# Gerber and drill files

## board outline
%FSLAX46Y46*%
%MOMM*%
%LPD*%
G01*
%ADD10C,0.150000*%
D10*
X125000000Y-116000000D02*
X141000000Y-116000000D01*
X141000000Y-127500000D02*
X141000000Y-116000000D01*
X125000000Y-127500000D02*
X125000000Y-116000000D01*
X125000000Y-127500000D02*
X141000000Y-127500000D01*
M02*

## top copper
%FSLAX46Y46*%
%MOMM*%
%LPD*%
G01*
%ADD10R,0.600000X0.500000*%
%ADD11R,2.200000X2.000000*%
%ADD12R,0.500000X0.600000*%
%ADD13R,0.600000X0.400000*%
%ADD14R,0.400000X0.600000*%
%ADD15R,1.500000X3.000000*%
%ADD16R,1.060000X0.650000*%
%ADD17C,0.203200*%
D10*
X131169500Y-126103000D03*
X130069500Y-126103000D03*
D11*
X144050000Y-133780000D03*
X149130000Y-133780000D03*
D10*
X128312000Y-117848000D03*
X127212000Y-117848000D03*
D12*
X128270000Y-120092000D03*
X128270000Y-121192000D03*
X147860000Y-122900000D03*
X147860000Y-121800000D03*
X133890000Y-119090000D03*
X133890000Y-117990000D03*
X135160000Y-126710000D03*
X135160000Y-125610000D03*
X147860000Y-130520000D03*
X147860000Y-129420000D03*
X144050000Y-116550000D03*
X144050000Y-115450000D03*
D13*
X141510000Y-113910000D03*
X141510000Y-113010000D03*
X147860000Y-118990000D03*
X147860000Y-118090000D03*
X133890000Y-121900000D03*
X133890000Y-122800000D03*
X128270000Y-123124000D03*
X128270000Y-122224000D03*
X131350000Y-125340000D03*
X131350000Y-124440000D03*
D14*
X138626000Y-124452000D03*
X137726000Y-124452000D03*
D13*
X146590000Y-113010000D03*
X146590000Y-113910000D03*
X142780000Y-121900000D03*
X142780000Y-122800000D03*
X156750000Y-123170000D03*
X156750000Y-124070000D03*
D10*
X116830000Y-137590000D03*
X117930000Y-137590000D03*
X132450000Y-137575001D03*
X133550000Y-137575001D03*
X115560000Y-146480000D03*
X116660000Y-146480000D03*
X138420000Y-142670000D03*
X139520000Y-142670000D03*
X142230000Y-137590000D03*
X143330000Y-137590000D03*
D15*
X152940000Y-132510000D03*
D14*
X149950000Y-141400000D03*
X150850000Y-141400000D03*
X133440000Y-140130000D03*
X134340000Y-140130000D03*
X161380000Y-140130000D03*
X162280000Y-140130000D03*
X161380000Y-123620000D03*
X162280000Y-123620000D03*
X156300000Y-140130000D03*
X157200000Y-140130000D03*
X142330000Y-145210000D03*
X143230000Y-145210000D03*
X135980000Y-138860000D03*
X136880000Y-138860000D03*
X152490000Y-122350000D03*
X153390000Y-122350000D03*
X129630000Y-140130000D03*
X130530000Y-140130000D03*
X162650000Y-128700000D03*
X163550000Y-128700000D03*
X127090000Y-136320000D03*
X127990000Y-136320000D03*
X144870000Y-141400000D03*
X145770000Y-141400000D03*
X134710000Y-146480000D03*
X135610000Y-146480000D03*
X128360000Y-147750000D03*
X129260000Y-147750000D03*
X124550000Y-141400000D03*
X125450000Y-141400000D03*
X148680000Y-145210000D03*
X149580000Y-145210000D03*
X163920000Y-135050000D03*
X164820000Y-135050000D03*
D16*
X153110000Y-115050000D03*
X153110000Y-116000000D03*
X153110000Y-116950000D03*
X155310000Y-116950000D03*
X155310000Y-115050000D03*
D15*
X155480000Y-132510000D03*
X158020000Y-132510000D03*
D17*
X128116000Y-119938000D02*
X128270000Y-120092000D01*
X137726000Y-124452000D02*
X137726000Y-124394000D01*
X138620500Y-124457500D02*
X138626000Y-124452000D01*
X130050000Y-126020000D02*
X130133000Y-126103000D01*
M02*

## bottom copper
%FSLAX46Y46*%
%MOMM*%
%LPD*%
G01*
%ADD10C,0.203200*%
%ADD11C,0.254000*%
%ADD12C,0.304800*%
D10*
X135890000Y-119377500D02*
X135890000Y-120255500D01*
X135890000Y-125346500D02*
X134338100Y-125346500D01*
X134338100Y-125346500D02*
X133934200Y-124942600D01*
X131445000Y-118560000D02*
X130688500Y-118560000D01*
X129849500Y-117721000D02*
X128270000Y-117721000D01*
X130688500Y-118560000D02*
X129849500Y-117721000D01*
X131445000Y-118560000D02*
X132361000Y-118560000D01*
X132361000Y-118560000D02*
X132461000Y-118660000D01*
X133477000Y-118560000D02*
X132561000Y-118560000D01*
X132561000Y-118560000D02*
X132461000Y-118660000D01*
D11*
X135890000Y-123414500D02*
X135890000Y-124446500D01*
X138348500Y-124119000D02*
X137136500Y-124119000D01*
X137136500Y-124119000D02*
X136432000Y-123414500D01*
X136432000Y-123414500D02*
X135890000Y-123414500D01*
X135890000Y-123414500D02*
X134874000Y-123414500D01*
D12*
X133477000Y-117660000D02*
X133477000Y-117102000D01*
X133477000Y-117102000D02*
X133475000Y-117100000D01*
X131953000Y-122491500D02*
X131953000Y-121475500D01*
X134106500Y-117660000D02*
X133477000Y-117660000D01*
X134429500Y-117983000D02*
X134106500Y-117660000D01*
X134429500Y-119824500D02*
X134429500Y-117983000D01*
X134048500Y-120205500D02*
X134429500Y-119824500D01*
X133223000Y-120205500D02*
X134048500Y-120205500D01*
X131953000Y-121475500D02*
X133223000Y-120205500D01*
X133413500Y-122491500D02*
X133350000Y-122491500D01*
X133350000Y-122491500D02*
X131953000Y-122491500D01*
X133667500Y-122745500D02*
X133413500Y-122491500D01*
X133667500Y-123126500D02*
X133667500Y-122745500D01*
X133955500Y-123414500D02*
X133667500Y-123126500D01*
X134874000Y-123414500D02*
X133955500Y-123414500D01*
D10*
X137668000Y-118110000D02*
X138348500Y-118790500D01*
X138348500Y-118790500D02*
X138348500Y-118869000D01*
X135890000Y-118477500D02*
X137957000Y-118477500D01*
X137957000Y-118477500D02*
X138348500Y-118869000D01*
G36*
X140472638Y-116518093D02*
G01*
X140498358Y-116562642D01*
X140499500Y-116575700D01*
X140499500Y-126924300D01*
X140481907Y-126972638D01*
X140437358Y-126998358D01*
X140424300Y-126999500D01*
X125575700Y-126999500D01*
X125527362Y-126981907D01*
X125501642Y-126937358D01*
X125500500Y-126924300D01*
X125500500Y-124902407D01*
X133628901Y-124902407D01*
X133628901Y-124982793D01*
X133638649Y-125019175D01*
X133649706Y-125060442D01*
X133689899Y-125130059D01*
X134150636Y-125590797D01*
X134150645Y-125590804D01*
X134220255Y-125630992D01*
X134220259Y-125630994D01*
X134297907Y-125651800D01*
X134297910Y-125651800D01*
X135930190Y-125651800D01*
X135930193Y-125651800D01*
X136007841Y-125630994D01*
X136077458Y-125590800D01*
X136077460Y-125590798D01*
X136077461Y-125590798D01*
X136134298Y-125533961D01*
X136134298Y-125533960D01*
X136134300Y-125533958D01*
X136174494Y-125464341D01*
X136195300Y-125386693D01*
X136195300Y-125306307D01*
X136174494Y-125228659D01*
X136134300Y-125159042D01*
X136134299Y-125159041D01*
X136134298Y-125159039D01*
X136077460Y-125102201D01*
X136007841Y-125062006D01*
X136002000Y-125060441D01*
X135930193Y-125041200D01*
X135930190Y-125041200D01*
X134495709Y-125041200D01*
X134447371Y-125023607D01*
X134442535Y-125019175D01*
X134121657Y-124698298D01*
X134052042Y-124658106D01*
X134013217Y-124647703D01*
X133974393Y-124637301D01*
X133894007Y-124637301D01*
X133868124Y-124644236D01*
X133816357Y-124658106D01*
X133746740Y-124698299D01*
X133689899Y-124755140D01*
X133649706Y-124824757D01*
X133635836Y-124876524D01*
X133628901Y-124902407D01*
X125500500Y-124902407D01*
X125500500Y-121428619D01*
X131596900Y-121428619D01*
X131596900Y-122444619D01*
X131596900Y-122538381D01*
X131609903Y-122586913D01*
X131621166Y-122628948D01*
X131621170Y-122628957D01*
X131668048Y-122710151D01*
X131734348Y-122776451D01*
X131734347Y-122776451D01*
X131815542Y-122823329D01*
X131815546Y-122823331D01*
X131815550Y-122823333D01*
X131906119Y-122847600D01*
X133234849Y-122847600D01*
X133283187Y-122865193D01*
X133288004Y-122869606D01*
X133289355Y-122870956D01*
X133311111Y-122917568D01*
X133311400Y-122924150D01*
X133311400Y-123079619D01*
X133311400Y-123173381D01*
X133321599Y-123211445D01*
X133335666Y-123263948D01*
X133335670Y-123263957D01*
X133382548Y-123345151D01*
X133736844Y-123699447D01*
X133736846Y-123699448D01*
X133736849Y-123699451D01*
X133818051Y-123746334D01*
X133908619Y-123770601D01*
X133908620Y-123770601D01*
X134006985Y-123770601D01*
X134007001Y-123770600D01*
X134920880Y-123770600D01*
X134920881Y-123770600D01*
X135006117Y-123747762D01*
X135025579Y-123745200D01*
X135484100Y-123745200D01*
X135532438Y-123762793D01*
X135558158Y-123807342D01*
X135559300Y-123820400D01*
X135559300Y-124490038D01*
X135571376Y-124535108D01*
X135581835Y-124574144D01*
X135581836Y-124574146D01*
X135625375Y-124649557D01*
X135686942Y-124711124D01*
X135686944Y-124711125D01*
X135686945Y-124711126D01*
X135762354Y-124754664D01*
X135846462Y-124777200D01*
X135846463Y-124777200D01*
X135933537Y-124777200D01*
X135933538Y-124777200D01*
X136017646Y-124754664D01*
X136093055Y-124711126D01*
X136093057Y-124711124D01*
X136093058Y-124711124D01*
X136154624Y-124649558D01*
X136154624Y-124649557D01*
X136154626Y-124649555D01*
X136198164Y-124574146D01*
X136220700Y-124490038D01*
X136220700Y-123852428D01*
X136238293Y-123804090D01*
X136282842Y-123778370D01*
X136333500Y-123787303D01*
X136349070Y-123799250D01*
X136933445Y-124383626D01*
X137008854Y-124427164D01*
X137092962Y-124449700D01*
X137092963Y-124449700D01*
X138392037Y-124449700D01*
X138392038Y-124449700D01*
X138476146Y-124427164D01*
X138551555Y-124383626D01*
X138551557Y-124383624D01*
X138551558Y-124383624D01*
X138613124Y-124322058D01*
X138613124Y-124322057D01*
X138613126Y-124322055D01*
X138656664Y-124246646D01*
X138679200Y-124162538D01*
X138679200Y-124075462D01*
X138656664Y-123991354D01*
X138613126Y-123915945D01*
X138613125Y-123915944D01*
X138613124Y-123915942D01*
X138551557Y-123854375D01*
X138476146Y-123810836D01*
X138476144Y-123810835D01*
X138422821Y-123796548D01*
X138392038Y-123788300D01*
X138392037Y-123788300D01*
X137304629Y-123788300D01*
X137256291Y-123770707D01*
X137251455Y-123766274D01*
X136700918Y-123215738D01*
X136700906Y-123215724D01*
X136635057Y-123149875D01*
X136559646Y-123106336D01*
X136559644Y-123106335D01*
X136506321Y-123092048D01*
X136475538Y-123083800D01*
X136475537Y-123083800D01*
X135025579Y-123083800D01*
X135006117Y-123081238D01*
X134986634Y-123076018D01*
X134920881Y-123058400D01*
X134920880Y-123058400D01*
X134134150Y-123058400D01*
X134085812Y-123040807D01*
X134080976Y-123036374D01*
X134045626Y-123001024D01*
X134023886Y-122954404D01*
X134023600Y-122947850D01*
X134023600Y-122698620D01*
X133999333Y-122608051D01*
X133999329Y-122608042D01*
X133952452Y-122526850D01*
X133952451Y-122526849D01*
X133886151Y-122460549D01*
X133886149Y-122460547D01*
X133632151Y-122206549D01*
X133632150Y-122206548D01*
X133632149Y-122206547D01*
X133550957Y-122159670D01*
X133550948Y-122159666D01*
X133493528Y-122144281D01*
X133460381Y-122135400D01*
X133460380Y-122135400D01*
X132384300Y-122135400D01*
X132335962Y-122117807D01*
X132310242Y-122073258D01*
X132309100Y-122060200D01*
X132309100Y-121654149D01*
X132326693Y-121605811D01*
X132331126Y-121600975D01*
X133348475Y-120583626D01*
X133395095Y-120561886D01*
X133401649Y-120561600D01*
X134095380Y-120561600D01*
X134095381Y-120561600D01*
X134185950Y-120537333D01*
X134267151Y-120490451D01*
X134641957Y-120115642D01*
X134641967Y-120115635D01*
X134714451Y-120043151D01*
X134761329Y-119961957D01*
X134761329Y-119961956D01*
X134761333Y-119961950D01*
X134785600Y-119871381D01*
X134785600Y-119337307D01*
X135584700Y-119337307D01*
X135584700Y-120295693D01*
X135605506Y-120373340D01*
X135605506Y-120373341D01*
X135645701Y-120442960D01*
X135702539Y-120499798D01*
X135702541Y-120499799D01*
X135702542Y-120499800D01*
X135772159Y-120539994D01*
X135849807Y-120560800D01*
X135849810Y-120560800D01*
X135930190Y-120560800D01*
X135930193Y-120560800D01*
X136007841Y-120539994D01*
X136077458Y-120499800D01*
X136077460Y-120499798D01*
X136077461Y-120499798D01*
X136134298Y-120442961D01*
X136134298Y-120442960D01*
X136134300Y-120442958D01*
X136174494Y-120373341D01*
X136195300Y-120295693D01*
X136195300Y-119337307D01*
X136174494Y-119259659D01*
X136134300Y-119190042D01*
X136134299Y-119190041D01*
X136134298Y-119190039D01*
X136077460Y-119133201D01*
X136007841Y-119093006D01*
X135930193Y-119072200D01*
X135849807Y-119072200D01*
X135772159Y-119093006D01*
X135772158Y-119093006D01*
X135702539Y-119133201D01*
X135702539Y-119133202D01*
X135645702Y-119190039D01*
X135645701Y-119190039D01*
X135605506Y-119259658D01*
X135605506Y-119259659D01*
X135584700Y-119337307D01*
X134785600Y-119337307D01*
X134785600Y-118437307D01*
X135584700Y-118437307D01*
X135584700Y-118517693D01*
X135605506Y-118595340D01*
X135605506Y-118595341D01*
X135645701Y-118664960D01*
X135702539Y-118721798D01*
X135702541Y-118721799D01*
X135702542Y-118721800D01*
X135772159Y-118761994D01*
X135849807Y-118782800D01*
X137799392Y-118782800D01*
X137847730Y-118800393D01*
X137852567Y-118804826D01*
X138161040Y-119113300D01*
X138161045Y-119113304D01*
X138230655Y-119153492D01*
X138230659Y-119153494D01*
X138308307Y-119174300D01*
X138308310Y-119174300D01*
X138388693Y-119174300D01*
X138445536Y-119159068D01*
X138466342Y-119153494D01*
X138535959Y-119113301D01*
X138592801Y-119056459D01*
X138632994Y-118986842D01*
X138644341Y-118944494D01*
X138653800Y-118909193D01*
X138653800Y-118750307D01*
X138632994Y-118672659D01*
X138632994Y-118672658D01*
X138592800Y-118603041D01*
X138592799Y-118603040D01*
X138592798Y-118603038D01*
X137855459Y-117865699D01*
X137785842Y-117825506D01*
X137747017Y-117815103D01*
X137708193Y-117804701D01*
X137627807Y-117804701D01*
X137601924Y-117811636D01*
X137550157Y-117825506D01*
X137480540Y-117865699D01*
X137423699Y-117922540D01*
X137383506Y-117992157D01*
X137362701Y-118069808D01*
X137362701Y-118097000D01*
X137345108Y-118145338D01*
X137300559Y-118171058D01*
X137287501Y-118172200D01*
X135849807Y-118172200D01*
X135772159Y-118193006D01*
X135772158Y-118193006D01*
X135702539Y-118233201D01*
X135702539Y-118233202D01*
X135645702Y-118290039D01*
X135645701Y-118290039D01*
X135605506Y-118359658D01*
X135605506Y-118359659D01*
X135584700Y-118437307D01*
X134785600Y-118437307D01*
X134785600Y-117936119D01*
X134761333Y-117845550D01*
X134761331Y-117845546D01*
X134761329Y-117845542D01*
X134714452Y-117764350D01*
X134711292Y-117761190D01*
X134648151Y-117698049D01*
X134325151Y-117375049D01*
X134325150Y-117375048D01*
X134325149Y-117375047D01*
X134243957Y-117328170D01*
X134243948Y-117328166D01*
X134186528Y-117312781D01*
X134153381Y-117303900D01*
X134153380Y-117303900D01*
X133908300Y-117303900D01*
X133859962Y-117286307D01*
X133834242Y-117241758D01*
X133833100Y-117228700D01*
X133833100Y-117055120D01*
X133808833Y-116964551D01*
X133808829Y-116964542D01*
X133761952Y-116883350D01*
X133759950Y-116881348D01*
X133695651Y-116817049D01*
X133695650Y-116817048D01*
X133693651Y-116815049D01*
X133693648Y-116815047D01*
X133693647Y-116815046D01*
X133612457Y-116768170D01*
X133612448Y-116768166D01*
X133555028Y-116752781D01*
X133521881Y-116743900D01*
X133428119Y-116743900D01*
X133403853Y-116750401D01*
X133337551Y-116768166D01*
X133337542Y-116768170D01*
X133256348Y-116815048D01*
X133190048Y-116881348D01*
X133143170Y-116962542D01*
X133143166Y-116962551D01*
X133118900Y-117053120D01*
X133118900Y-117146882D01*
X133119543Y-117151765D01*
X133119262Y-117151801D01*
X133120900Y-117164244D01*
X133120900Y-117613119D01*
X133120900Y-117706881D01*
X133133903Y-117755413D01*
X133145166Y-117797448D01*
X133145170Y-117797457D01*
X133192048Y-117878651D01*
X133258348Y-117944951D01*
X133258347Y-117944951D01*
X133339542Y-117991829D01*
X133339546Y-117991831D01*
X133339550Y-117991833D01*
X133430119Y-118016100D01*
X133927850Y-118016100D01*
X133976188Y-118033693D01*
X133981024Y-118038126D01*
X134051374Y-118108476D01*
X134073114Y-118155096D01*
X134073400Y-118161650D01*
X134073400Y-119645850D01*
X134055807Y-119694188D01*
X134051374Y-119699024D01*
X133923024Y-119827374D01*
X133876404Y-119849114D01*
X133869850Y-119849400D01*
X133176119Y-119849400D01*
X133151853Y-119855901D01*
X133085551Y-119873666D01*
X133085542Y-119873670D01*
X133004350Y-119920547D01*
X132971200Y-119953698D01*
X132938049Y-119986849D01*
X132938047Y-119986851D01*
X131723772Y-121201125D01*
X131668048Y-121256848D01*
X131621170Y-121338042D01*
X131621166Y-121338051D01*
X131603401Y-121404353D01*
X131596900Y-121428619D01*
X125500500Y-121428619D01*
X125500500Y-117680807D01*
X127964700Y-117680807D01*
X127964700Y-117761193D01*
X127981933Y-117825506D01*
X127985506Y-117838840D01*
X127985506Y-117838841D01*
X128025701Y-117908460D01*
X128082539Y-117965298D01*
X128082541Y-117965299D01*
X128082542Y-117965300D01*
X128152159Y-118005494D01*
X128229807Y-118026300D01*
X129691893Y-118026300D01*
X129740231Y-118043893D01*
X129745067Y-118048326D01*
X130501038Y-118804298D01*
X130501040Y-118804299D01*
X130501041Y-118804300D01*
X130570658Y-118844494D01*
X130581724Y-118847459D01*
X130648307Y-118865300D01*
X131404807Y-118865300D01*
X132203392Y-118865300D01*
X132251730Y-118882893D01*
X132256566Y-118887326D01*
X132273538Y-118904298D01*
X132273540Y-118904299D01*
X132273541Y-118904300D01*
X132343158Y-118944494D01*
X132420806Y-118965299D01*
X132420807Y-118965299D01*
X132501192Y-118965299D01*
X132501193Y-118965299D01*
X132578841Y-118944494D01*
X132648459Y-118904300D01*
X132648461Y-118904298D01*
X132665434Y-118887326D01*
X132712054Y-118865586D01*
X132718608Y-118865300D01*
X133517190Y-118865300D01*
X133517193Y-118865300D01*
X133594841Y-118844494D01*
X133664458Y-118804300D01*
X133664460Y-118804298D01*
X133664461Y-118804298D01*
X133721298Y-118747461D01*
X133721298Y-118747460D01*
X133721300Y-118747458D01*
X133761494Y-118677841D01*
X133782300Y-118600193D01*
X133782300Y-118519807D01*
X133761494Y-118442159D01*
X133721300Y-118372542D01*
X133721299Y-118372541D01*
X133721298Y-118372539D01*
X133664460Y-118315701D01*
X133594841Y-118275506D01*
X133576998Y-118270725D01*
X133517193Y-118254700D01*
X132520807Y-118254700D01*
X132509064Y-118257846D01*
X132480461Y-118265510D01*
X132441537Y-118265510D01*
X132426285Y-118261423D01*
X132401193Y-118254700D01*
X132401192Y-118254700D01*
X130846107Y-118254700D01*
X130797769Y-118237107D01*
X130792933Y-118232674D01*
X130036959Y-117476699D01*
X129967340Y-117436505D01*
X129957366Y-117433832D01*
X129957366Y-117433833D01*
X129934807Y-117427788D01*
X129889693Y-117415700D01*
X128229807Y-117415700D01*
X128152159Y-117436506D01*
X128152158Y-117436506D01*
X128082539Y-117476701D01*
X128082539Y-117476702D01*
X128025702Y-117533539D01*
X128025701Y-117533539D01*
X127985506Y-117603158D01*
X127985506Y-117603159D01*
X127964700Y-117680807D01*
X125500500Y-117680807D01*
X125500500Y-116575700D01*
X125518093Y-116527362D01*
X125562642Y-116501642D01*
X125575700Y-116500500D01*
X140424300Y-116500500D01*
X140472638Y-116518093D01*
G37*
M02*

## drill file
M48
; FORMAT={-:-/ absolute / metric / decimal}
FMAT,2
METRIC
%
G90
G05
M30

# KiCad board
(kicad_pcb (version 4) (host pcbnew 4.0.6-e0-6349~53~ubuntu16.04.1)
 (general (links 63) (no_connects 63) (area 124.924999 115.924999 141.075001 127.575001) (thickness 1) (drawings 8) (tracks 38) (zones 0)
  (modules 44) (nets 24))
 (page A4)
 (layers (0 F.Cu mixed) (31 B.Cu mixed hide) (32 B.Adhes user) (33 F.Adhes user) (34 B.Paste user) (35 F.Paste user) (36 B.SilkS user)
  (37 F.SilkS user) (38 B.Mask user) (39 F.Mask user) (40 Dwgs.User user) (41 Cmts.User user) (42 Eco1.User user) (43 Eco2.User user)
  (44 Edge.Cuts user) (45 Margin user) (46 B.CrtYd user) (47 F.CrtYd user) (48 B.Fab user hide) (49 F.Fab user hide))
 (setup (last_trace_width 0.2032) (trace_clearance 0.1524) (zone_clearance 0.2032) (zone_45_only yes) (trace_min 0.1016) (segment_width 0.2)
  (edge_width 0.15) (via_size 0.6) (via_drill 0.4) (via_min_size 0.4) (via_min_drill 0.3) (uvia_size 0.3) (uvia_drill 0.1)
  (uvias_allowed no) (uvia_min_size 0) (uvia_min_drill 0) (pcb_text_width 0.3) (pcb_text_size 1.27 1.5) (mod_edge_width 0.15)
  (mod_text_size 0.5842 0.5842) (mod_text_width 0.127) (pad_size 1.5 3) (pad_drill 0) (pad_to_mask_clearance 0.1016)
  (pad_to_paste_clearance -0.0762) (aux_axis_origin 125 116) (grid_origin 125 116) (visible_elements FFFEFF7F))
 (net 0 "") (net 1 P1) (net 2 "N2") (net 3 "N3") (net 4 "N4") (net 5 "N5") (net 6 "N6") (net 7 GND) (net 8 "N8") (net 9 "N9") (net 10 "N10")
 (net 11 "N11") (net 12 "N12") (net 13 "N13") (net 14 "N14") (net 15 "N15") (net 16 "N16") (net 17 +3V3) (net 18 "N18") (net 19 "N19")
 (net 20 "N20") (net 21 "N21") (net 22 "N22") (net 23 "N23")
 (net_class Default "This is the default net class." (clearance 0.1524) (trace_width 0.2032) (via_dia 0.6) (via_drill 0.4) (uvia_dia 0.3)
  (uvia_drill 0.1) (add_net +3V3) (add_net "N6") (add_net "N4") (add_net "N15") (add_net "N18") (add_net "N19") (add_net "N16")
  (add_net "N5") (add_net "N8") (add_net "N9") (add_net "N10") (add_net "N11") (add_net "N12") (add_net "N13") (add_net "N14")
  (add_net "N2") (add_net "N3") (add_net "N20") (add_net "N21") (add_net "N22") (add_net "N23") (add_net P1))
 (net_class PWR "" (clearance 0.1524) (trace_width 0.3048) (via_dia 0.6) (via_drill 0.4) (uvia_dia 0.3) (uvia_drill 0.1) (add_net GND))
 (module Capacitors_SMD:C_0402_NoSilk (layer F.Cu) (at 130.6195 126.103 180)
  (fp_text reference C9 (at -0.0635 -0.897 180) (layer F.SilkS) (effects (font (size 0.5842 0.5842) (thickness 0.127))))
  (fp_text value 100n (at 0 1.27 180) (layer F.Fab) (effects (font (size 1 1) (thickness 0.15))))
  (pad 1 smd rect (at -0.55 0 180) (size 0.6 0.5) (layers F.Cu F.Paste F.Mask) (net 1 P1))
  (pad 2 smd rect (at 0.55 0 180) (size 0.6 0.5) (layers F.Cu F.Paste F.Mask) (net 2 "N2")))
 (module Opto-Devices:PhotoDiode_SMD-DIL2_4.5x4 (layer F.Cu) (at 146.59 133.78 180)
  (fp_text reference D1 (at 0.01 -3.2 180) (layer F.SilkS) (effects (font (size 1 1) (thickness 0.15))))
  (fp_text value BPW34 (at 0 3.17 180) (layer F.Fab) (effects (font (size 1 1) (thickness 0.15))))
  (pad 2 smd rect (at 2.54 0) (size 2.2 2) (layers F.Cu F.Paste F.Mask) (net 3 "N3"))
  (pad 1 smd rect (at -2.54 0) (size 2.2 2) (layers F.Cu F.Paste F.Mask) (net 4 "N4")))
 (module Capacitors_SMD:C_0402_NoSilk (layer F.Cu) (at 127.762 117.848 180)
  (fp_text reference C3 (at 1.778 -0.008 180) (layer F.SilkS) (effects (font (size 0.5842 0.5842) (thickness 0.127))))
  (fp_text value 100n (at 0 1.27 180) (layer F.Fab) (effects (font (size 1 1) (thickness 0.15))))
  (pad 1 smd rect (at -0.55 0 180) (size 0.6 0.5) (layers F.Cu F.Paste F.Mask) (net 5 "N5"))
  (pad 2 smd rect (at 0.55 0 180) (size 0.6 0.5) (layers F.Cu F.Paste F.Mask) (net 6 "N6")))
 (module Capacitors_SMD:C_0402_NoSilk (layer F.Cu) (at 128.27 120.642 270)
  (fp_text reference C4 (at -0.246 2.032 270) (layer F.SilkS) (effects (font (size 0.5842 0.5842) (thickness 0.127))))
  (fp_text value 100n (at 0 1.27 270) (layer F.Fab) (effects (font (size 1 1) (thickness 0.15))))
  (pad 1 smd rect (at -0.55 0 270) (size 0.6 0.5) (layers F.Cu F.Paste F.Mask) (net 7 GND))
  (pad 2 smd rect (at 0.55 0 270) (size 0.6 0.5) (layers F.Cu F.Paste F.Mask) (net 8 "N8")))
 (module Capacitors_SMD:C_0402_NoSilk (layer F.Cu) (at 147.86 122.35 90)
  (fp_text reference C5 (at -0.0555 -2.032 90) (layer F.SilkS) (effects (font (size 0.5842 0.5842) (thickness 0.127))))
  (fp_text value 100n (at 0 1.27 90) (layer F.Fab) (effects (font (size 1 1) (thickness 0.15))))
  (pad 1 smd rect (at -0.55 0 90) (size 0.6 0.5) (layers F.Cu F.Paste F.Mask) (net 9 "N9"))
  (pad 2 smd rect (at 0.55 0 90) (size 0.6 0.5) (layers F.Cu F.Paste F.Mask) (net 7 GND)))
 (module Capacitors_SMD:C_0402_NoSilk (layer F.Cu) (at 133.89 118.54 90)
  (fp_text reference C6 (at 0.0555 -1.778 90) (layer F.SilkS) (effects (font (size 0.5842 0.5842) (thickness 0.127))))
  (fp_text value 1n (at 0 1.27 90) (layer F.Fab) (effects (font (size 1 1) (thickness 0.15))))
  (pad 1 smd rect (at -0.55 0 90) (size 0.6 0.5) (layers F.Cu F.Paste F.Mask) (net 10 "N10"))
  (pad 2 smd rect (at 0.55 0 90) (size 0.6 0.5) (layers F.Cu F.Paste F.Mask) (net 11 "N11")))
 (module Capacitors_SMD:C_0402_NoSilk (layer F.Cu) (at 135.16 126.16 90)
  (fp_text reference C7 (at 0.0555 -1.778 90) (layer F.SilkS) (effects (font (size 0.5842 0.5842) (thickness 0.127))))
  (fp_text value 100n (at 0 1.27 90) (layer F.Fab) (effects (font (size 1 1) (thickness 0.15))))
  (pad 1 smd rect (at -0.55 0 90) (size 0.6 0.5) (layers F.Cu F.Paste F.Mask) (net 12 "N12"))
  (pad 2 smd rect (at 0.55 0 90) (size 0.6 0.5) (layers F.Cu F.Paste F.Mask) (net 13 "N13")))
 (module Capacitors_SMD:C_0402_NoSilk (layer F.Cu) (at 147.86 129.97 90)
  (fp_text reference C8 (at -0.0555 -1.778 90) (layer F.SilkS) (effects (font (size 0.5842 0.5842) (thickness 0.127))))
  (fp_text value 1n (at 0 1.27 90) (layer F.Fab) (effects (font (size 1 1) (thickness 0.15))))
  (pad 1 smd rect (at -0.55 0 90) (size 0.6 0.5) (layers F.Cu F.Paste F.Mask) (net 7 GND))
  (pad 2 smd rect (at 0.55 0 90) (size 0.6 0.5) (layers F.Cu F.Paste F.Mask) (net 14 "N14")))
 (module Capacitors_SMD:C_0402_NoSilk (layer F.Cu) (at 144.05 116 90)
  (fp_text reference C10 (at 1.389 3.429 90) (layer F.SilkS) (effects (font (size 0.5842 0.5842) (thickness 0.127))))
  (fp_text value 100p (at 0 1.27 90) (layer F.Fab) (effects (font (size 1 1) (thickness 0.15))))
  (pad 1 smd rect (at -0.55 0 90) (size 0.6 0.5) (layers F.Cu F.Paste F.Mask) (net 7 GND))
  (pad 2 smd rect (at 0.55 0 90) (size 0.6 0.5) (layers F.Cu F.Paste F.Mask) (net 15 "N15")))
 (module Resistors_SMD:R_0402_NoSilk (layer F.Cu) (at 141.51 113.46 90)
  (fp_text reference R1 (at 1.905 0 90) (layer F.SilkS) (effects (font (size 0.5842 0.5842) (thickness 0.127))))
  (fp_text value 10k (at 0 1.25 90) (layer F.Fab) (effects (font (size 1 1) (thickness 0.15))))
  (pad 1 smd rect (at -0.45 0 90) (size 0.4 0.6) (layers F.Cu F.Paste F.Mask) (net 8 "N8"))
  (pad 2 smd rect (at 0.45 0 90) (size 0.4 0.6) (layers F.Cu F.Paste F.Mask) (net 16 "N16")))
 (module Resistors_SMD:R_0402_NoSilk (layer F.Cu) (at 147.86 118.54 90)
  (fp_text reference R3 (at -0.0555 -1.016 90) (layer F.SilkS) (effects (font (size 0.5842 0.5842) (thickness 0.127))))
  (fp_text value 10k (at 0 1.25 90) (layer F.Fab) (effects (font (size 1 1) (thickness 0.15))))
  (pad 1 smd rect (at -0.45 0 90) (size 0.4 0.6) (layers F.Cu F.Paste F.Mask) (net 16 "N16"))
  (pad 2 smd rect (at 0.45 0 90) (size 0.4 0.6) (layers F.Cu F.Paste F.Mask) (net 4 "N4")))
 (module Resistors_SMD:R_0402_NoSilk (layer F.Cu) (at 133.89 122.35 270)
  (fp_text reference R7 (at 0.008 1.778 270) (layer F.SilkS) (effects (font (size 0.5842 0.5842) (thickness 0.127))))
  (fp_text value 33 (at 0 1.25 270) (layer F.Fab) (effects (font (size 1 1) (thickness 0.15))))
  (pad 1 smd rect (at -0.45 0 270) (size 0.4 0.6) (layers F.Cu F.Paste F.Mask) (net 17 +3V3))
  (pad 2 smd rect (at 0.45 0 270) (size 0.4 0.6) (layers F.Cu F.Paste F.Mask) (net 8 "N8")))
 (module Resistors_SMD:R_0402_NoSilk (layer F.Cu) (at 128.27 122.674 90)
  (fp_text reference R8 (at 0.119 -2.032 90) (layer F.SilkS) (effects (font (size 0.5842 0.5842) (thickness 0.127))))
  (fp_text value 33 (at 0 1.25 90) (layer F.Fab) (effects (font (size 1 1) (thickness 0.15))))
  (pad 1 smd rect (at -0.45 0 90) (size 0.4 0.6) (layers F.Cu F.Paste F.Mask) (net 17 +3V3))
  (pad 2 smd rect (at 0.45 0 90) (size 0.4 0.6) (layers F.Cu F.Paste F.Mask) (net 9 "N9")))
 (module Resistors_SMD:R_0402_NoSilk (layer F.Cu) (at 131.35 124.89 90)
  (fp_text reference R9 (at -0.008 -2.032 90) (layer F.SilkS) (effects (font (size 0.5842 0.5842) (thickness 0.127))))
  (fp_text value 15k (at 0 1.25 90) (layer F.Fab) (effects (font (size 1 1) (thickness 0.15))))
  (pad 1 smd rect (at -0.45 0 90) (size 0.4 0.6) (layers F.Cu F.Paste F.Mask) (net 9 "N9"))
  (pad 2 smd rect (at 0.45 0 90) (size 0.4 0.6) (layers F.Cu F.Paste F.Mask) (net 5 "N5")))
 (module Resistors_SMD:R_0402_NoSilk (layer F.Cu) (at 138.176 124.452 180)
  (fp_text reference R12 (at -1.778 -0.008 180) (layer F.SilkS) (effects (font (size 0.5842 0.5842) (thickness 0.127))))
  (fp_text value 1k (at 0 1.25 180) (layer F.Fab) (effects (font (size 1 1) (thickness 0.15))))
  (pad 1 smd rect (at -0.45 0 180) (size 0.4 0.6) (layers F.Cu F.Paste F.Mask) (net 11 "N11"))
  (pad 2 smd rect (at 0.45 0 180) (size 0.4 0.6) (layers F.Cu F.Paste F.Mask) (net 10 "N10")))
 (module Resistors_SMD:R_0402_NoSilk (layer F.Cu) (at 146.59 113.46 270)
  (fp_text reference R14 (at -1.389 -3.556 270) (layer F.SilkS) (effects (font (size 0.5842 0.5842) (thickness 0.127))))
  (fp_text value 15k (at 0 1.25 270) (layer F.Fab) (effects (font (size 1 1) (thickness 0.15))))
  (pad 1 smd rect (at -0.45 0 270) (size 0.4 0.6) (layers F.Cu F.Paste F.Mask) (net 12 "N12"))
  (pad 2 smd rect (at 0.45 0 270) (size 0.4 0.6) (layers F.Cu F.Paste F.Mask) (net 10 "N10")))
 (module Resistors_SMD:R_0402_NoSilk (layer F.Cu) (at 142.78 122.35 270)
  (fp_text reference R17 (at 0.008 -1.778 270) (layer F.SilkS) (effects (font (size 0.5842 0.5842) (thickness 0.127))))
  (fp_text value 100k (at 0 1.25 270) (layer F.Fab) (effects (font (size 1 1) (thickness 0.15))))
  (pad 1 smd rect (at -0.45 0 270) (size 0.4 0.6) (layers F.Cu F.Paste F.Mask) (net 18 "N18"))
  (pad 2 smd rect (at 0.45 0 270) (size 0.4 0.6) (layers F.Cu F.Paste F.Mask) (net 1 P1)))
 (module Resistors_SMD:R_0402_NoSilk (layer F.Cu) (at 156.75 123.62 270)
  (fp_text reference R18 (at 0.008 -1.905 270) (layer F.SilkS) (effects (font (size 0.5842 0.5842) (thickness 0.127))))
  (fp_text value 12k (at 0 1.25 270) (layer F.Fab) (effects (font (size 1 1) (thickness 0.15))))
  (pad 1 smd rect (at -0.45 0 270) (size 0.4 0.6) (layers F.Cu F.Paste F.Mask) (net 1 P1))
  (pad 2 smd rect (at 0.45 0 270) (size 0.4 0.6) (layers F.Cu F.Paste F.Mask) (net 7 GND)))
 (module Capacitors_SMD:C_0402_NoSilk (layer F.Cu) (at 117.38 137.59)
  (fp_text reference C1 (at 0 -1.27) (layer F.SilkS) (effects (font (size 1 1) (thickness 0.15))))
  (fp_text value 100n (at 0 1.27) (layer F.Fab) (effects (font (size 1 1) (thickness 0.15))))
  (pad 1 smd rect (at -0.55 0) (size 0.6 0.5) (layers F.Cu F.Paste F.Mask) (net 6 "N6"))
  (pad 2 smd rect (at 0.55 0) (size 0.6 0.5) (layers F.Cu F.Paste F.Mask) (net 4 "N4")))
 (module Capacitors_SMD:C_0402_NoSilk (layer F.Cu) (at 133 137.575001)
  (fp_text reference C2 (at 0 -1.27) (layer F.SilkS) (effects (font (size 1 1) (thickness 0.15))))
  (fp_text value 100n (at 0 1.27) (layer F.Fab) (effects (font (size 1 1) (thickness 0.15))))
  (pad 1 smd rect (at -0.55 0) (size 0.6 0.5) (layers F.Cu F.Paste F.Mask) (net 16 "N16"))
  (pad 2 smd rect (at 0.55 0) (size 0.6 0.5) (layers F.Cu F.Paste F.Mask) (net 7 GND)))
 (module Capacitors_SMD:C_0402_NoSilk (layer F.Cu) (at 116.11 146.48)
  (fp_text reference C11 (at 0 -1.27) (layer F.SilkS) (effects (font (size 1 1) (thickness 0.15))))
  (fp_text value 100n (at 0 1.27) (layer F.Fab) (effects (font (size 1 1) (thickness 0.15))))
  (pad 1 smd rect (at -0.55 0) (size 0.6 0.5) (layers F.Cu F.Paste F.Mask) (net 7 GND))
  (pad 2 smd rect (at 0.55 0) (size 0.6 0.5) (layers F.Cu F.Paste F.Mask) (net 18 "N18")))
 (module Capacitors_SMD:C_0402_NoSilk (layer F.Cu) (at 138.97 142.67)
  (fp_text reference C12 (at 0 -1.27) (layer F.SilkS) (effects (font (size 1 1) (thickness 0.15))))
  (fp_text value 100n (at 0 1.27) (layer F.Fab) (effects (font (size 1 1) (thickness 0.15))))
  (pad 1 smd rect (at -0.55 0) (size 0.6 0.5) (layers F.Cu F.Paste F.Mask) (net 7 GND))
  (pad 2 smd rect (at 0.55 0) (size 0.6 0.5) (layers F.Cu F.Paste F.Mask) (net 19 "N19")))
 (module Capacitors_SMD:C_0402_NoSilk (layer F.Cu) (at 142.78 137.59)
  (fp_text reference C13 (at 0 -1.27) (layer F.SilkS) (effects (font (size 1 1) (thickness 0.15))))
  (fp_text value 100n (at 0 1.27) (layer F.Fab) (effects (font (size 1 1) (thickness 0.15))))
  (pad 1 smd rect (at -0.55 0) (size 0.6 0.5) (layers F.Cu F.Paste F.Mask) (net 7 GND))
  (pad 2 smd rect (at 0.55 0) (size 0.6 0.5) (layers F.Cu F.Paste F.Mask) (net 17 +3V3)))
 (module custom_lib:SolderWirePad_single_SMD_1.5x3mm (layer F.Cu) (at 152.94 132.51)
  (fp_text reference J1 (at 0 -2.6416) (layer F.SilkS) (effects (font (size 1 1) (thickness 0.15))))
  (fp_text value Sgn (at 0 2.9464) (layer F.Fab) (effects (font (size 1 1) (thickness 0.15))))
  (pad 1 smd rect (at 0 0) (size 1.5 3) (layers F.Cu F.Paste F.Mask) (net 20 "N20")))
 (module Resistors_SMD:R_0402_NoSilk (layer F.Cu) (at 150.4 141.4)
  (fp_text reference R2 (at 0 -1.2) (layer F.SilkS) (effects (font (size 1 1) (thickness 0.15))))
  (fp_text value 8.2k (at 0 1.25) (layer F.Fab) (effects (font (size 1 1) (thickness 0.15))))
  (pad 1 smd rect (at -0.45 0) (size 0.4 0.6) (layers F.Cu F.Paste F.Mask) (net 8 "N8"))
  (pad 2 smd rect (at 0.45 0) (size 0.4 0.6) (layers F.Cu F.Paste F.Mask) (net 3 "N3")))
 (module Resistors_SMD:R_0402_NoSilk (layer F.Cu) (at 133.89 140.13)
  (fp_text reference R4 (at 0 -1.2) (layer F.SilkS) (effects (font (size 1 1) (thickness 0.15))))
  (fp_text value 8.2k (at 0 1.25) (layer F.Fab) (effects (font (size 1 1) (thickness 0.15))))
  (pad 1 smd rect (at -0.45 0) (size 0.4 0.6) (layers F.Cu F.Paste F.Mask) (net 3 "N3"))
  (pad 2 smd rect (at 0.45 0) (size 0.4 0.6) (layers F.Cu F.Paste F.Mask) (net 7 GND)))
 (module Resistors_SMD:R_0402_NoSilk (layer F.Cu) (at 161.83 140.13)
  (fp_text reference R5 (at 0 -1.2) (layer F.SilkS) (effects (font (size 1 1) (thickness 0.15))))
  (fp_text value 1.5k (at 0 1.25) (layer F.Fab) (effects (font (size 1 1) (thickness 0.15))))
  (pad 1 smd rect (at -0.45 0) (size 0.4 0.6) (layers F.Cu F.Paste F.Mask) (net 8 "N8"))
  (pad 2 smd rect (at 0.45 0) (size 0.4 0.6) (layers F.Cu F.Paste F.Mask)))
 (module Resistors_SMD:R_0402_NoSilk (layer F.Cu) (at 161.83 123.62)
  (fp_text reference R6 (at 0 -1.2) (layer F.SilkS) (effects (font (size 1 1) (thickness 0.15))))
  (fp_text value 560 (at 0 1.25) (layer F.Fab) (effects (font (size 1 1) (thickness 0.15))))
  (pad 1 smd rect (at -0.45 0) (size 0.4 0.6) (layers F.Cu F.Paste F.Mask) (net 6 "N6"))
  (pad 2 smd rect (at 0.45 0) (size 0.4 0.6) (layers F.Cu F.Paste F.Mask) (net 7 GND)))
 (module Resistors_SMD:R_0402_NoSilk (layer F.Cu) (at 156.75 140.13)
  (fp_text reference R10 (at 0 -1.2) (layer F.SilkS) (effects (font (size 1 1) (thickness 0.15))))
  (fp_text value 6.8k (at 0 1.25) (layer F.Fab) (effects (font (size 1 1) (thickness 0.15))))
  (pad 1 smd rect (at -0.45 0) (size 0.4 0.6) (layers F.Cu F.Paste F.Mask) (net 5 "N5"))
  (pad 2 smd rect (at 0.45 0) (size 0.4 0.6) (layers F.Cu F.Paste F.Mask) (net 10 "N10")))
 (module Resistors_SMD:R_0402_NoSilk (layer F.Cu) (at 142.78 145.21)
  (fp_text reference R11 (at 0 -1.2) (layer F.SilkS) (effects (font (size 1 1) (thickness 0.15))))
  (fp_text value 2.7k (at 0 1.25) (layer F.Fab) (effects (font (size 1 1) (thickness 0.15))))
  (pad 1 smd rect (at -0.45 0) (size 0.4 0.6) (layers F.Cu F.Paste F.Mask) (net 9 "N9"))
  (pad 2 smd rect (at 0.45 0) (size 0.4 0.6) (layers F.Cu F.Paste F.Mask) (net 13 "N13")))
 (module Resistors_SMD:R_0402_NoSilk (layer F.Cu) (at 136.43 138.86)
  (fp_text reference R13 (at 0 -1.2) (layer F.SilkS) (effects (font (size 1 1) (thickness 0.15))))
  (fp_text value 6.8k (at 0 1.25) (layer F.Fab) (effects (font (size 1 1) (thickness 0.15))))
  (pad 1 smd rect (at -0.45 0) (size 0.4 0.6) (layers F.Cu F.Paste F.Mask) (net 9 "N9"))
  (pad 2 smd rect (at 0.45 0) (size 0.4 0.6) (layers F.Cu F.Paste F.Mask) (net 12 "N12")))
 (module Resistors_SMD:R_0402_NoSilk (layer F.Cu) (at 152.94 122.35)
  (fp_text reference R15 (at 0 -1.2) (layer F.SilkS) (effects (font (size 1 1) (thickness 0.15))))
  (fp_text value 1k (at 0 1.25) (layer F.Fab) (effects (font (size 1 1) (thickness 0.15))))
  (pad 1 smd rect (at -0.45 0) (size 0.4 0.6) (layers F.Cu F.Paste F.Mask) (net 9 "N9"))
  (pad 2 smd rect (at 0.45 0) (size 0.4 0.6) (layers F.Cu F.Paste F.Mask) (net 14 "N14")))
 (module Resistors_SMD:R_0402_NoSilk (layer F.Cu) (at 130.08 140.13)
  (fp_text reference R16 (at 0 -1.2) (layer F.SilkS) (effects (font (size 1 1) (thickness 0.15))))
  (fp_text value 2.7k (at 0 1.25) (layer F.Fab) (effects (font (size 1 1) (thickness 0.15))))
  (pad 1 smd rect (at -0.45 0) (size 0.4 0.6) (layers F.Cu F.Paste F.Mask) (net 2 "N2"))
  (pad 2 smd rect (at 0.45 0) (size 0.4 0.6) (layers F.Cu F.Paste F.Mask) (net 10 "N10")))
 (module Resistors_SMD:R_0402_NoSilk (layer F.Cu) (at 163.1 128.7)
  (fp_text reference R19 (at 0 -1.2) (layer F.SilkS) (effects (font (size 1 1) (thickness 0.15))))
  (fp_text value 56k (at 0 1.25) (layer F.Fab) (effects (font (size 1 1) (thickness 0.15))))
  (pad 1 smd rect (at -0.45 0) (size 0.4 0.6) (layers F.Cu F.Paste F.Mask) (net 15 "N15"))
  (pad 2 smd rect (at 0.45 0) (size 0.4 0.6) (layers F.Cu F.Paste F.Mask)))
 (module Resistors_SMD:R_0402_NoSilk (layer F.Cu) (at 127.54 136.32)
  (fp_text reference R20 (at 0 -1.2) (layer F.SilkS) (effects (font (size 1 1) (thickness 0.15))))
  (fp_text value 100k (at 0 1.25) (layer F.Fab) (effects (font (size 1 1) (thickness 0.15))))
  (pad 1 smd rect (at -0.45 0) (size 0.4 0.6) (layers F.Cu F.Paste F.Mask) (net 18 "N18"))
  (pad 2 smd rect (at 0.45 0) (size 0.4 0.6) (layers F.Cu F.Paste F.Mask) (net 15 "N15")))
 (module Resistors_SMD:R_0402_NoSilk (layer F.Cu) (at 145.32 141.4)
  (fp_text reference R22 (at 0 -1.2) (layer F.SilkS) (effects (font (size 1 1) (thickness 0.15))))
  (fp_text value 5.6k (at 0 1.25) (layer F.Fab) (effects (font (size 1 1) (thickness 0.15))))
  (pad 1 smd rect (at -0.45 0) (size 0.4 0.6) (layers F.Cu F.Paste F.Mask) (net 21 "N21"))
  (pad 2 smd rect (at 0.45 0) (size 0.4 0.6) (layers F.Cu F.Paste F.Mask) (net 7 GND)))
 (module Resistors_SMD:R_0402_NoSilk (layer F.Cu) (at 135.16 146.48)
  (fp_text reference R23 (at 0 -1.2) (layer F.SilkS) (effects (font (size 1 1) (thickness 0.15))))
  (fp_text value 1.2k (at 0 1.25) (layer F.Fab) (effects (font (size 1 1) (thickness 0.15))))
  (pad 1 smd rect (at -0.45 0) (size 0.4 0.6) (layers F.Cu F.Paste F.Mask) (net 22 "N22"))
  (pad 2 smd rect (at 0.45 0) (size 0.4 0.6) (layers F.Cu F.Paste F.Mask) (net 21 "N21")))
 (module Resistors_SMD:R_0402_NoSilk (layer F.Cu) (at 128.81 147.75)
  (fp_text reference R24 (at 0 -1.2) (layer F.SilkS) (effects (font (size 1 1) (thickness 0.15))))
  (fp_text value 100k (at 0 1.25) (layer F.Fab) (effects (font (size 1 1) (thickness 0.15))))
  (pad 1 smd rect (at -0.45 0) (size 0.4 0.6) (layers F.Cu F.Paste F.Mask) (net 17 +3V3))
  (pad 2 smd rect (at 0.45 0) (size 0.4 0.6) (layers F.Cu F.Paste F.Mask) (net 19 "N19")))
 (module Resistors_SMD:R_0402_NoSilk (layer F.Cu) (at 125 141.4)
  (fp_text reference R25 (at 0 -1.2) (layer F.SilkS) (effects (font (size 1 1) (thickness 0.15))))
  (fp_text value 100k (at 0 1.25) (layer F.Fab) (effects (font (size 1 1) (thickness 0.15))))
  (pad 1 smd rect (at -0.45 0) (size 0.4 0.6) (layers F.Cu F.Paste F.Mask) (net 19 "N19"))
  (pad 2 smd rect (at 0.45 0) (size 0.4 0.6) (layers F.Cu F.Paste F.Mask) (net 7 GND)))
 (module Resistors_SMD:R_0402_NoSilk (layer F.Cu) (at 149.13 145.21)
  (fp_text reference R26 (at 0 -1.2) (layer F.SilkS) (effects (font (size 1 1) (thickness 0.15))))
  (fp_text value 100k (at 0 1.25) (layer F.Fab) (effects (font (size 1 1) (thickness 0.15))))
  (pad 1 smd rect (at -0.45 0) (size 0.4 0.6) (layers F.Cu F.Paste F.Mask) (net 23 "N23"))
  (pad 2 smd rect (at 0.45 0) (size 0.4 0.6) (layers F.Cu F.Paste F.Mask) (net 22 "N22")))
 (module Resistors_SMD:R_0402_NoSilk (layer F.Cu) (at 164.37 135.05)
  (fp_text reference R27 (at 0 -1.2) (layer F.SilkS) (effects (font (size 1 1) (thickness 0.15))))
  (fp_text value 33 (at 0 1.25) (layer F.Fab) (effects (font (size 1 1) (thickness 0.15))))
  (pad 1 smd rect (at -0.45 0) (size 0.4 0.6) (layers F.Cu F.Paste F.Mask) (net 20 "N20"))
  (pad 2 smd rect (at 0.45 0) (size 0.4 0.6) (layers F.Cu F.Paste F.Mask) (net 23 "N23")))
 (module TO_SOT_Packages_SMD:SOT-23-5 (layer F.Cu) (at 154.21 116)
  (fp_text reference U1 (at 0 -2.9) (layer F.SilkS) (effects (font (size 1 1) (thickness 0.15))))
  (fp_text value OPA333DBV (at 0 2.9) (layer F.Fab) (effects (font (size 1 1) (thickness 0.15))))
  (pad 1 smd rect (at -1.1 -0.95) (size 1.06 0.65) (layers F.Cu F.Paste F.Mask) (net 23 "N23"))
  (pad 2 smd rect (at -1.1 0) (size 1.06 0.65) (layers F.Cu F.Paste F.Mask) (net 7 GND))
  (pad 3 smd rect (at -1.1 0.95) (size 1.06 0.65) (layers F.Cu F.Paste F.Mask) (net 22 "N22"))
  (pad 4 smd rect (at 1.1 0.95) (size 1.06 0.65) (layers F.Cu F.Paste F.Mask) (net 19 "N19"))
  (pad 5 smd rect (at 1.1 -0.95) (size 1.06 0.65) (layers F.Cu F.Paste F.Mask) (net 17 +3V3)))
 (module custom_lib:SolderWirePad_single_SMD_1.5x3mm (layer F.Cu) (at 155.48 132.51)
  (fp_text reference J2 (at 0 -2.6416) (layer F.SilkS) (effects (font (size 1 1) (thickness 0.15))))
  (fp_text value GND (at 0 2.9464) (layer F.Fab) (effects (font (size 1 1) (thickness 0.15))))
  (pad 1 smd rect (at 0 0) (size 1.5 3) (layers F.Cu F.Paste F.Mask) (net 7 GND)))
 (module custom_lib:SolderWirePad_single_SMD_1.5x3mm (layer F.Cu) (at 158.02 132.51)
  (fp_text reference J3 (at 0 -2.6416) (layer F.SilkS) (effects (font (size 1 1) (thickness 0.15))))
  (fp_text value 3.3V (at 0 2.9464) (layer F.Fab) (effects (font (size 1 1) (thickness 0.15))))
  (pad 1 smd rect (at 0 0) (size 1.5 3) (layers F.Cu F.Paste F.Mask) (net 17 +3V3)))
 (gr_line (start 125 116) (end 141 116) (angle 90) (layer Edge.Cuts) (width 0.15))
 (gr_line (start 141 127.5) (end 141 116) (angle 90) (layer Edge.Cuts) (width 0.15))
 (gr_line (start 125 127.5) (end 125 116) (angle 90) (layer Edge.Cuts) (width 0.15))
 (gr_line (start 125 127.5) (end 141 127.5) (angle 90) (layer Edge.Cuts) (width 0.15))
 (segment (start 135.89 119.3775) (end 135.89 120.2555) (width 0.2032) (layer B.Cu) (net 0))
 (segment (start 135.89 125.3465) (end 134.3381 125.3465) (width 0.2032) (layer B.Cu) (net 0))
 (segment (start 134.3381 125.3465) (end 133.9342 124.9426) (width 0.2032) (layer B.Cu) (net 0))
 (segment (start 131.445 118.56) (end 130.6885 118.56) (width 0.2032) (layer B.Cu) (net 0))
 (segment (start 129.8495 117.721) (end 128.27 117.721) (width 0.2032) (layer B.Cu) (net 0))
 (segment (start 130.6885 118.56) (end 129.8495 117.721) (width 0.2032) (layer B.Cu) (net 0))
 (segment (start 131.445 118.56) (end 132.361 118.56) (width 0.2032) (layer B.Cu) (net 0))
 (segment (start 132.361 118.56) (end 132.461 118.66) (width 0.2032) (layer B.Cu) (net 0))
 (segment (start 133.477 118.56) (end 132.561 118.56) (width 0.2032) (layer B.Cu) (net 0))
 (segment (start 132.561 118.56) (end 132.461 118.66) (width 0.2032) (layer B.Cu) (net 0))
 (segment (start 135.89 123.4145) (end 135.89 124.4465) (width 0.254) (layer B.Cu) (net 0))
 (segment (start 138.3485 124.119) (end 137.1365 124.119) (width 0.254) (layer B.Cu) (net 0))
 (segment (start 137.1365 124.119) (end 136.432 123.4145) (width 0.254) (layer B.Cu) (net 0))
 (segment (start 136.432 123.4145) (end 135.89 123.4145) (width 0.254) (layer B.Cu) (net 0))
 (segment (start 135.89 123.4145) (end 134.874 123.4145) (width 0.254) (layer B.Cu) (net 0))
 (segment (start 133.477 117.66) (end 133.477 117.102) (width 0.3048) (layer B.Cu) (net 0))
 (segment (start 133.477 117.102) (end 133.475 117.1) (width 0.3048) (layer B.Cu) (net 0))
 (segment (start 131.953 122.4915) (end 131.953 121.4755) (width 0.3048) (layer B.Cu) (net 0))
 (segment (start 134.1065 117.66) (end 133.477 117.66) (width 0.3048) (layer B.Cu) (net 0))
 (segment (start 134.4295 117.983) (end 134.1065 117.66) (width 0.3048) (layer B.Cu) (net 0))
 (segment (start 134.4295 119.8245) (end 134.4295 117.983) (width 0.3048) (layer B.Cu) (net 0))
 (segment (start 134.0485 120.2055) (end 134.4295 119.8245) (width 0.3048) (layer B.Cu) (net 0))
 (segment (start 133.223 120.2055) (end 134.0485 120.2055) (width 0.3048) (layer B.Cu) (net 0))
 (segment (start 131.953 121.4755) (end 133.223 120.2055) (width 0.3048) (layer B.Cu) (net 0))
 (segment (start 133.4135 122.4915) (end 133.35 122.4915) (width 0.3048) (layer B.Cu) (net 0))
 (segment (start 133.35 122.4915) (end 131.953 122.4915) (width 0.3048) (layer B.Cu) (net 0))
 (segment (start 133.6675 122.7455) (end 133.4135 122.4915) (width 0.3048) (layer B.Cu) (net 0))
 (segment (start 133.6675 123.1265) (end 133.6675 122.7455) (width 0.3048) (layer B.Cu) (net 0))
 (segment (start 133.9555 123.4145) (end 133.6675 123.1265) (width 0.3048) (layer B.Cu) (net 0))
 (segment (start 134.874 123.4145) (end 133.9555 123.4145) (width 0.3048) (layer B.Cu) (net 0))
 (segment (start 137.668 118.11) (end 138.3485 118.7905) (width 0.2032) (layer B.Cu) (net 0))
 (segment (start 138.3485 118.7905) (end 138.3485 118.869) (width 0.2032) (layer B.Cu) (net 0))
 (segment (start 135.89 118.4775) (end 137.957 118.4775) (width 0.2032) (layer B.Cu) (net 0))
 (segment (start 137.957 118.4775) (end 138.3485 118.869) (width 0.2032) (layer B.Cu) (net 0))
 (segment (start 128.116 119.938) (end 128.27 120.092) (width 0.2032) (layer F.Cu) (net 7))
 (segment (start 137.726 124.452) (end 137.726 124.394) (width 0.2032) (layer F.Cu) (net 10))
 (segment (start 138.6205 124.4575) (end 138.626 124.452) (width 0.2032) (layer F.Cu) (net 11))
 (segment (start 130.05 126.02) (end 130.133 126.103) (width 0.2032) (layer F.Cu) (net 2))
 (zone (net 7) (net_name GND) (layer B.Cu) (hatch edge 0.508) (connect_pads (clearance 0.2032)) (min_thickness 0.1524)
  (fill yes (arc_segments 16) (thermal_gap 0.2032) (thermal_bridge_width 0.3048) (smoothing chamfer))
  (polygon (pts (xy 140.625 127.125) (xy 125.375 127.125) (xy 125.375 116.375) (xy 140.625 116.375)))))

